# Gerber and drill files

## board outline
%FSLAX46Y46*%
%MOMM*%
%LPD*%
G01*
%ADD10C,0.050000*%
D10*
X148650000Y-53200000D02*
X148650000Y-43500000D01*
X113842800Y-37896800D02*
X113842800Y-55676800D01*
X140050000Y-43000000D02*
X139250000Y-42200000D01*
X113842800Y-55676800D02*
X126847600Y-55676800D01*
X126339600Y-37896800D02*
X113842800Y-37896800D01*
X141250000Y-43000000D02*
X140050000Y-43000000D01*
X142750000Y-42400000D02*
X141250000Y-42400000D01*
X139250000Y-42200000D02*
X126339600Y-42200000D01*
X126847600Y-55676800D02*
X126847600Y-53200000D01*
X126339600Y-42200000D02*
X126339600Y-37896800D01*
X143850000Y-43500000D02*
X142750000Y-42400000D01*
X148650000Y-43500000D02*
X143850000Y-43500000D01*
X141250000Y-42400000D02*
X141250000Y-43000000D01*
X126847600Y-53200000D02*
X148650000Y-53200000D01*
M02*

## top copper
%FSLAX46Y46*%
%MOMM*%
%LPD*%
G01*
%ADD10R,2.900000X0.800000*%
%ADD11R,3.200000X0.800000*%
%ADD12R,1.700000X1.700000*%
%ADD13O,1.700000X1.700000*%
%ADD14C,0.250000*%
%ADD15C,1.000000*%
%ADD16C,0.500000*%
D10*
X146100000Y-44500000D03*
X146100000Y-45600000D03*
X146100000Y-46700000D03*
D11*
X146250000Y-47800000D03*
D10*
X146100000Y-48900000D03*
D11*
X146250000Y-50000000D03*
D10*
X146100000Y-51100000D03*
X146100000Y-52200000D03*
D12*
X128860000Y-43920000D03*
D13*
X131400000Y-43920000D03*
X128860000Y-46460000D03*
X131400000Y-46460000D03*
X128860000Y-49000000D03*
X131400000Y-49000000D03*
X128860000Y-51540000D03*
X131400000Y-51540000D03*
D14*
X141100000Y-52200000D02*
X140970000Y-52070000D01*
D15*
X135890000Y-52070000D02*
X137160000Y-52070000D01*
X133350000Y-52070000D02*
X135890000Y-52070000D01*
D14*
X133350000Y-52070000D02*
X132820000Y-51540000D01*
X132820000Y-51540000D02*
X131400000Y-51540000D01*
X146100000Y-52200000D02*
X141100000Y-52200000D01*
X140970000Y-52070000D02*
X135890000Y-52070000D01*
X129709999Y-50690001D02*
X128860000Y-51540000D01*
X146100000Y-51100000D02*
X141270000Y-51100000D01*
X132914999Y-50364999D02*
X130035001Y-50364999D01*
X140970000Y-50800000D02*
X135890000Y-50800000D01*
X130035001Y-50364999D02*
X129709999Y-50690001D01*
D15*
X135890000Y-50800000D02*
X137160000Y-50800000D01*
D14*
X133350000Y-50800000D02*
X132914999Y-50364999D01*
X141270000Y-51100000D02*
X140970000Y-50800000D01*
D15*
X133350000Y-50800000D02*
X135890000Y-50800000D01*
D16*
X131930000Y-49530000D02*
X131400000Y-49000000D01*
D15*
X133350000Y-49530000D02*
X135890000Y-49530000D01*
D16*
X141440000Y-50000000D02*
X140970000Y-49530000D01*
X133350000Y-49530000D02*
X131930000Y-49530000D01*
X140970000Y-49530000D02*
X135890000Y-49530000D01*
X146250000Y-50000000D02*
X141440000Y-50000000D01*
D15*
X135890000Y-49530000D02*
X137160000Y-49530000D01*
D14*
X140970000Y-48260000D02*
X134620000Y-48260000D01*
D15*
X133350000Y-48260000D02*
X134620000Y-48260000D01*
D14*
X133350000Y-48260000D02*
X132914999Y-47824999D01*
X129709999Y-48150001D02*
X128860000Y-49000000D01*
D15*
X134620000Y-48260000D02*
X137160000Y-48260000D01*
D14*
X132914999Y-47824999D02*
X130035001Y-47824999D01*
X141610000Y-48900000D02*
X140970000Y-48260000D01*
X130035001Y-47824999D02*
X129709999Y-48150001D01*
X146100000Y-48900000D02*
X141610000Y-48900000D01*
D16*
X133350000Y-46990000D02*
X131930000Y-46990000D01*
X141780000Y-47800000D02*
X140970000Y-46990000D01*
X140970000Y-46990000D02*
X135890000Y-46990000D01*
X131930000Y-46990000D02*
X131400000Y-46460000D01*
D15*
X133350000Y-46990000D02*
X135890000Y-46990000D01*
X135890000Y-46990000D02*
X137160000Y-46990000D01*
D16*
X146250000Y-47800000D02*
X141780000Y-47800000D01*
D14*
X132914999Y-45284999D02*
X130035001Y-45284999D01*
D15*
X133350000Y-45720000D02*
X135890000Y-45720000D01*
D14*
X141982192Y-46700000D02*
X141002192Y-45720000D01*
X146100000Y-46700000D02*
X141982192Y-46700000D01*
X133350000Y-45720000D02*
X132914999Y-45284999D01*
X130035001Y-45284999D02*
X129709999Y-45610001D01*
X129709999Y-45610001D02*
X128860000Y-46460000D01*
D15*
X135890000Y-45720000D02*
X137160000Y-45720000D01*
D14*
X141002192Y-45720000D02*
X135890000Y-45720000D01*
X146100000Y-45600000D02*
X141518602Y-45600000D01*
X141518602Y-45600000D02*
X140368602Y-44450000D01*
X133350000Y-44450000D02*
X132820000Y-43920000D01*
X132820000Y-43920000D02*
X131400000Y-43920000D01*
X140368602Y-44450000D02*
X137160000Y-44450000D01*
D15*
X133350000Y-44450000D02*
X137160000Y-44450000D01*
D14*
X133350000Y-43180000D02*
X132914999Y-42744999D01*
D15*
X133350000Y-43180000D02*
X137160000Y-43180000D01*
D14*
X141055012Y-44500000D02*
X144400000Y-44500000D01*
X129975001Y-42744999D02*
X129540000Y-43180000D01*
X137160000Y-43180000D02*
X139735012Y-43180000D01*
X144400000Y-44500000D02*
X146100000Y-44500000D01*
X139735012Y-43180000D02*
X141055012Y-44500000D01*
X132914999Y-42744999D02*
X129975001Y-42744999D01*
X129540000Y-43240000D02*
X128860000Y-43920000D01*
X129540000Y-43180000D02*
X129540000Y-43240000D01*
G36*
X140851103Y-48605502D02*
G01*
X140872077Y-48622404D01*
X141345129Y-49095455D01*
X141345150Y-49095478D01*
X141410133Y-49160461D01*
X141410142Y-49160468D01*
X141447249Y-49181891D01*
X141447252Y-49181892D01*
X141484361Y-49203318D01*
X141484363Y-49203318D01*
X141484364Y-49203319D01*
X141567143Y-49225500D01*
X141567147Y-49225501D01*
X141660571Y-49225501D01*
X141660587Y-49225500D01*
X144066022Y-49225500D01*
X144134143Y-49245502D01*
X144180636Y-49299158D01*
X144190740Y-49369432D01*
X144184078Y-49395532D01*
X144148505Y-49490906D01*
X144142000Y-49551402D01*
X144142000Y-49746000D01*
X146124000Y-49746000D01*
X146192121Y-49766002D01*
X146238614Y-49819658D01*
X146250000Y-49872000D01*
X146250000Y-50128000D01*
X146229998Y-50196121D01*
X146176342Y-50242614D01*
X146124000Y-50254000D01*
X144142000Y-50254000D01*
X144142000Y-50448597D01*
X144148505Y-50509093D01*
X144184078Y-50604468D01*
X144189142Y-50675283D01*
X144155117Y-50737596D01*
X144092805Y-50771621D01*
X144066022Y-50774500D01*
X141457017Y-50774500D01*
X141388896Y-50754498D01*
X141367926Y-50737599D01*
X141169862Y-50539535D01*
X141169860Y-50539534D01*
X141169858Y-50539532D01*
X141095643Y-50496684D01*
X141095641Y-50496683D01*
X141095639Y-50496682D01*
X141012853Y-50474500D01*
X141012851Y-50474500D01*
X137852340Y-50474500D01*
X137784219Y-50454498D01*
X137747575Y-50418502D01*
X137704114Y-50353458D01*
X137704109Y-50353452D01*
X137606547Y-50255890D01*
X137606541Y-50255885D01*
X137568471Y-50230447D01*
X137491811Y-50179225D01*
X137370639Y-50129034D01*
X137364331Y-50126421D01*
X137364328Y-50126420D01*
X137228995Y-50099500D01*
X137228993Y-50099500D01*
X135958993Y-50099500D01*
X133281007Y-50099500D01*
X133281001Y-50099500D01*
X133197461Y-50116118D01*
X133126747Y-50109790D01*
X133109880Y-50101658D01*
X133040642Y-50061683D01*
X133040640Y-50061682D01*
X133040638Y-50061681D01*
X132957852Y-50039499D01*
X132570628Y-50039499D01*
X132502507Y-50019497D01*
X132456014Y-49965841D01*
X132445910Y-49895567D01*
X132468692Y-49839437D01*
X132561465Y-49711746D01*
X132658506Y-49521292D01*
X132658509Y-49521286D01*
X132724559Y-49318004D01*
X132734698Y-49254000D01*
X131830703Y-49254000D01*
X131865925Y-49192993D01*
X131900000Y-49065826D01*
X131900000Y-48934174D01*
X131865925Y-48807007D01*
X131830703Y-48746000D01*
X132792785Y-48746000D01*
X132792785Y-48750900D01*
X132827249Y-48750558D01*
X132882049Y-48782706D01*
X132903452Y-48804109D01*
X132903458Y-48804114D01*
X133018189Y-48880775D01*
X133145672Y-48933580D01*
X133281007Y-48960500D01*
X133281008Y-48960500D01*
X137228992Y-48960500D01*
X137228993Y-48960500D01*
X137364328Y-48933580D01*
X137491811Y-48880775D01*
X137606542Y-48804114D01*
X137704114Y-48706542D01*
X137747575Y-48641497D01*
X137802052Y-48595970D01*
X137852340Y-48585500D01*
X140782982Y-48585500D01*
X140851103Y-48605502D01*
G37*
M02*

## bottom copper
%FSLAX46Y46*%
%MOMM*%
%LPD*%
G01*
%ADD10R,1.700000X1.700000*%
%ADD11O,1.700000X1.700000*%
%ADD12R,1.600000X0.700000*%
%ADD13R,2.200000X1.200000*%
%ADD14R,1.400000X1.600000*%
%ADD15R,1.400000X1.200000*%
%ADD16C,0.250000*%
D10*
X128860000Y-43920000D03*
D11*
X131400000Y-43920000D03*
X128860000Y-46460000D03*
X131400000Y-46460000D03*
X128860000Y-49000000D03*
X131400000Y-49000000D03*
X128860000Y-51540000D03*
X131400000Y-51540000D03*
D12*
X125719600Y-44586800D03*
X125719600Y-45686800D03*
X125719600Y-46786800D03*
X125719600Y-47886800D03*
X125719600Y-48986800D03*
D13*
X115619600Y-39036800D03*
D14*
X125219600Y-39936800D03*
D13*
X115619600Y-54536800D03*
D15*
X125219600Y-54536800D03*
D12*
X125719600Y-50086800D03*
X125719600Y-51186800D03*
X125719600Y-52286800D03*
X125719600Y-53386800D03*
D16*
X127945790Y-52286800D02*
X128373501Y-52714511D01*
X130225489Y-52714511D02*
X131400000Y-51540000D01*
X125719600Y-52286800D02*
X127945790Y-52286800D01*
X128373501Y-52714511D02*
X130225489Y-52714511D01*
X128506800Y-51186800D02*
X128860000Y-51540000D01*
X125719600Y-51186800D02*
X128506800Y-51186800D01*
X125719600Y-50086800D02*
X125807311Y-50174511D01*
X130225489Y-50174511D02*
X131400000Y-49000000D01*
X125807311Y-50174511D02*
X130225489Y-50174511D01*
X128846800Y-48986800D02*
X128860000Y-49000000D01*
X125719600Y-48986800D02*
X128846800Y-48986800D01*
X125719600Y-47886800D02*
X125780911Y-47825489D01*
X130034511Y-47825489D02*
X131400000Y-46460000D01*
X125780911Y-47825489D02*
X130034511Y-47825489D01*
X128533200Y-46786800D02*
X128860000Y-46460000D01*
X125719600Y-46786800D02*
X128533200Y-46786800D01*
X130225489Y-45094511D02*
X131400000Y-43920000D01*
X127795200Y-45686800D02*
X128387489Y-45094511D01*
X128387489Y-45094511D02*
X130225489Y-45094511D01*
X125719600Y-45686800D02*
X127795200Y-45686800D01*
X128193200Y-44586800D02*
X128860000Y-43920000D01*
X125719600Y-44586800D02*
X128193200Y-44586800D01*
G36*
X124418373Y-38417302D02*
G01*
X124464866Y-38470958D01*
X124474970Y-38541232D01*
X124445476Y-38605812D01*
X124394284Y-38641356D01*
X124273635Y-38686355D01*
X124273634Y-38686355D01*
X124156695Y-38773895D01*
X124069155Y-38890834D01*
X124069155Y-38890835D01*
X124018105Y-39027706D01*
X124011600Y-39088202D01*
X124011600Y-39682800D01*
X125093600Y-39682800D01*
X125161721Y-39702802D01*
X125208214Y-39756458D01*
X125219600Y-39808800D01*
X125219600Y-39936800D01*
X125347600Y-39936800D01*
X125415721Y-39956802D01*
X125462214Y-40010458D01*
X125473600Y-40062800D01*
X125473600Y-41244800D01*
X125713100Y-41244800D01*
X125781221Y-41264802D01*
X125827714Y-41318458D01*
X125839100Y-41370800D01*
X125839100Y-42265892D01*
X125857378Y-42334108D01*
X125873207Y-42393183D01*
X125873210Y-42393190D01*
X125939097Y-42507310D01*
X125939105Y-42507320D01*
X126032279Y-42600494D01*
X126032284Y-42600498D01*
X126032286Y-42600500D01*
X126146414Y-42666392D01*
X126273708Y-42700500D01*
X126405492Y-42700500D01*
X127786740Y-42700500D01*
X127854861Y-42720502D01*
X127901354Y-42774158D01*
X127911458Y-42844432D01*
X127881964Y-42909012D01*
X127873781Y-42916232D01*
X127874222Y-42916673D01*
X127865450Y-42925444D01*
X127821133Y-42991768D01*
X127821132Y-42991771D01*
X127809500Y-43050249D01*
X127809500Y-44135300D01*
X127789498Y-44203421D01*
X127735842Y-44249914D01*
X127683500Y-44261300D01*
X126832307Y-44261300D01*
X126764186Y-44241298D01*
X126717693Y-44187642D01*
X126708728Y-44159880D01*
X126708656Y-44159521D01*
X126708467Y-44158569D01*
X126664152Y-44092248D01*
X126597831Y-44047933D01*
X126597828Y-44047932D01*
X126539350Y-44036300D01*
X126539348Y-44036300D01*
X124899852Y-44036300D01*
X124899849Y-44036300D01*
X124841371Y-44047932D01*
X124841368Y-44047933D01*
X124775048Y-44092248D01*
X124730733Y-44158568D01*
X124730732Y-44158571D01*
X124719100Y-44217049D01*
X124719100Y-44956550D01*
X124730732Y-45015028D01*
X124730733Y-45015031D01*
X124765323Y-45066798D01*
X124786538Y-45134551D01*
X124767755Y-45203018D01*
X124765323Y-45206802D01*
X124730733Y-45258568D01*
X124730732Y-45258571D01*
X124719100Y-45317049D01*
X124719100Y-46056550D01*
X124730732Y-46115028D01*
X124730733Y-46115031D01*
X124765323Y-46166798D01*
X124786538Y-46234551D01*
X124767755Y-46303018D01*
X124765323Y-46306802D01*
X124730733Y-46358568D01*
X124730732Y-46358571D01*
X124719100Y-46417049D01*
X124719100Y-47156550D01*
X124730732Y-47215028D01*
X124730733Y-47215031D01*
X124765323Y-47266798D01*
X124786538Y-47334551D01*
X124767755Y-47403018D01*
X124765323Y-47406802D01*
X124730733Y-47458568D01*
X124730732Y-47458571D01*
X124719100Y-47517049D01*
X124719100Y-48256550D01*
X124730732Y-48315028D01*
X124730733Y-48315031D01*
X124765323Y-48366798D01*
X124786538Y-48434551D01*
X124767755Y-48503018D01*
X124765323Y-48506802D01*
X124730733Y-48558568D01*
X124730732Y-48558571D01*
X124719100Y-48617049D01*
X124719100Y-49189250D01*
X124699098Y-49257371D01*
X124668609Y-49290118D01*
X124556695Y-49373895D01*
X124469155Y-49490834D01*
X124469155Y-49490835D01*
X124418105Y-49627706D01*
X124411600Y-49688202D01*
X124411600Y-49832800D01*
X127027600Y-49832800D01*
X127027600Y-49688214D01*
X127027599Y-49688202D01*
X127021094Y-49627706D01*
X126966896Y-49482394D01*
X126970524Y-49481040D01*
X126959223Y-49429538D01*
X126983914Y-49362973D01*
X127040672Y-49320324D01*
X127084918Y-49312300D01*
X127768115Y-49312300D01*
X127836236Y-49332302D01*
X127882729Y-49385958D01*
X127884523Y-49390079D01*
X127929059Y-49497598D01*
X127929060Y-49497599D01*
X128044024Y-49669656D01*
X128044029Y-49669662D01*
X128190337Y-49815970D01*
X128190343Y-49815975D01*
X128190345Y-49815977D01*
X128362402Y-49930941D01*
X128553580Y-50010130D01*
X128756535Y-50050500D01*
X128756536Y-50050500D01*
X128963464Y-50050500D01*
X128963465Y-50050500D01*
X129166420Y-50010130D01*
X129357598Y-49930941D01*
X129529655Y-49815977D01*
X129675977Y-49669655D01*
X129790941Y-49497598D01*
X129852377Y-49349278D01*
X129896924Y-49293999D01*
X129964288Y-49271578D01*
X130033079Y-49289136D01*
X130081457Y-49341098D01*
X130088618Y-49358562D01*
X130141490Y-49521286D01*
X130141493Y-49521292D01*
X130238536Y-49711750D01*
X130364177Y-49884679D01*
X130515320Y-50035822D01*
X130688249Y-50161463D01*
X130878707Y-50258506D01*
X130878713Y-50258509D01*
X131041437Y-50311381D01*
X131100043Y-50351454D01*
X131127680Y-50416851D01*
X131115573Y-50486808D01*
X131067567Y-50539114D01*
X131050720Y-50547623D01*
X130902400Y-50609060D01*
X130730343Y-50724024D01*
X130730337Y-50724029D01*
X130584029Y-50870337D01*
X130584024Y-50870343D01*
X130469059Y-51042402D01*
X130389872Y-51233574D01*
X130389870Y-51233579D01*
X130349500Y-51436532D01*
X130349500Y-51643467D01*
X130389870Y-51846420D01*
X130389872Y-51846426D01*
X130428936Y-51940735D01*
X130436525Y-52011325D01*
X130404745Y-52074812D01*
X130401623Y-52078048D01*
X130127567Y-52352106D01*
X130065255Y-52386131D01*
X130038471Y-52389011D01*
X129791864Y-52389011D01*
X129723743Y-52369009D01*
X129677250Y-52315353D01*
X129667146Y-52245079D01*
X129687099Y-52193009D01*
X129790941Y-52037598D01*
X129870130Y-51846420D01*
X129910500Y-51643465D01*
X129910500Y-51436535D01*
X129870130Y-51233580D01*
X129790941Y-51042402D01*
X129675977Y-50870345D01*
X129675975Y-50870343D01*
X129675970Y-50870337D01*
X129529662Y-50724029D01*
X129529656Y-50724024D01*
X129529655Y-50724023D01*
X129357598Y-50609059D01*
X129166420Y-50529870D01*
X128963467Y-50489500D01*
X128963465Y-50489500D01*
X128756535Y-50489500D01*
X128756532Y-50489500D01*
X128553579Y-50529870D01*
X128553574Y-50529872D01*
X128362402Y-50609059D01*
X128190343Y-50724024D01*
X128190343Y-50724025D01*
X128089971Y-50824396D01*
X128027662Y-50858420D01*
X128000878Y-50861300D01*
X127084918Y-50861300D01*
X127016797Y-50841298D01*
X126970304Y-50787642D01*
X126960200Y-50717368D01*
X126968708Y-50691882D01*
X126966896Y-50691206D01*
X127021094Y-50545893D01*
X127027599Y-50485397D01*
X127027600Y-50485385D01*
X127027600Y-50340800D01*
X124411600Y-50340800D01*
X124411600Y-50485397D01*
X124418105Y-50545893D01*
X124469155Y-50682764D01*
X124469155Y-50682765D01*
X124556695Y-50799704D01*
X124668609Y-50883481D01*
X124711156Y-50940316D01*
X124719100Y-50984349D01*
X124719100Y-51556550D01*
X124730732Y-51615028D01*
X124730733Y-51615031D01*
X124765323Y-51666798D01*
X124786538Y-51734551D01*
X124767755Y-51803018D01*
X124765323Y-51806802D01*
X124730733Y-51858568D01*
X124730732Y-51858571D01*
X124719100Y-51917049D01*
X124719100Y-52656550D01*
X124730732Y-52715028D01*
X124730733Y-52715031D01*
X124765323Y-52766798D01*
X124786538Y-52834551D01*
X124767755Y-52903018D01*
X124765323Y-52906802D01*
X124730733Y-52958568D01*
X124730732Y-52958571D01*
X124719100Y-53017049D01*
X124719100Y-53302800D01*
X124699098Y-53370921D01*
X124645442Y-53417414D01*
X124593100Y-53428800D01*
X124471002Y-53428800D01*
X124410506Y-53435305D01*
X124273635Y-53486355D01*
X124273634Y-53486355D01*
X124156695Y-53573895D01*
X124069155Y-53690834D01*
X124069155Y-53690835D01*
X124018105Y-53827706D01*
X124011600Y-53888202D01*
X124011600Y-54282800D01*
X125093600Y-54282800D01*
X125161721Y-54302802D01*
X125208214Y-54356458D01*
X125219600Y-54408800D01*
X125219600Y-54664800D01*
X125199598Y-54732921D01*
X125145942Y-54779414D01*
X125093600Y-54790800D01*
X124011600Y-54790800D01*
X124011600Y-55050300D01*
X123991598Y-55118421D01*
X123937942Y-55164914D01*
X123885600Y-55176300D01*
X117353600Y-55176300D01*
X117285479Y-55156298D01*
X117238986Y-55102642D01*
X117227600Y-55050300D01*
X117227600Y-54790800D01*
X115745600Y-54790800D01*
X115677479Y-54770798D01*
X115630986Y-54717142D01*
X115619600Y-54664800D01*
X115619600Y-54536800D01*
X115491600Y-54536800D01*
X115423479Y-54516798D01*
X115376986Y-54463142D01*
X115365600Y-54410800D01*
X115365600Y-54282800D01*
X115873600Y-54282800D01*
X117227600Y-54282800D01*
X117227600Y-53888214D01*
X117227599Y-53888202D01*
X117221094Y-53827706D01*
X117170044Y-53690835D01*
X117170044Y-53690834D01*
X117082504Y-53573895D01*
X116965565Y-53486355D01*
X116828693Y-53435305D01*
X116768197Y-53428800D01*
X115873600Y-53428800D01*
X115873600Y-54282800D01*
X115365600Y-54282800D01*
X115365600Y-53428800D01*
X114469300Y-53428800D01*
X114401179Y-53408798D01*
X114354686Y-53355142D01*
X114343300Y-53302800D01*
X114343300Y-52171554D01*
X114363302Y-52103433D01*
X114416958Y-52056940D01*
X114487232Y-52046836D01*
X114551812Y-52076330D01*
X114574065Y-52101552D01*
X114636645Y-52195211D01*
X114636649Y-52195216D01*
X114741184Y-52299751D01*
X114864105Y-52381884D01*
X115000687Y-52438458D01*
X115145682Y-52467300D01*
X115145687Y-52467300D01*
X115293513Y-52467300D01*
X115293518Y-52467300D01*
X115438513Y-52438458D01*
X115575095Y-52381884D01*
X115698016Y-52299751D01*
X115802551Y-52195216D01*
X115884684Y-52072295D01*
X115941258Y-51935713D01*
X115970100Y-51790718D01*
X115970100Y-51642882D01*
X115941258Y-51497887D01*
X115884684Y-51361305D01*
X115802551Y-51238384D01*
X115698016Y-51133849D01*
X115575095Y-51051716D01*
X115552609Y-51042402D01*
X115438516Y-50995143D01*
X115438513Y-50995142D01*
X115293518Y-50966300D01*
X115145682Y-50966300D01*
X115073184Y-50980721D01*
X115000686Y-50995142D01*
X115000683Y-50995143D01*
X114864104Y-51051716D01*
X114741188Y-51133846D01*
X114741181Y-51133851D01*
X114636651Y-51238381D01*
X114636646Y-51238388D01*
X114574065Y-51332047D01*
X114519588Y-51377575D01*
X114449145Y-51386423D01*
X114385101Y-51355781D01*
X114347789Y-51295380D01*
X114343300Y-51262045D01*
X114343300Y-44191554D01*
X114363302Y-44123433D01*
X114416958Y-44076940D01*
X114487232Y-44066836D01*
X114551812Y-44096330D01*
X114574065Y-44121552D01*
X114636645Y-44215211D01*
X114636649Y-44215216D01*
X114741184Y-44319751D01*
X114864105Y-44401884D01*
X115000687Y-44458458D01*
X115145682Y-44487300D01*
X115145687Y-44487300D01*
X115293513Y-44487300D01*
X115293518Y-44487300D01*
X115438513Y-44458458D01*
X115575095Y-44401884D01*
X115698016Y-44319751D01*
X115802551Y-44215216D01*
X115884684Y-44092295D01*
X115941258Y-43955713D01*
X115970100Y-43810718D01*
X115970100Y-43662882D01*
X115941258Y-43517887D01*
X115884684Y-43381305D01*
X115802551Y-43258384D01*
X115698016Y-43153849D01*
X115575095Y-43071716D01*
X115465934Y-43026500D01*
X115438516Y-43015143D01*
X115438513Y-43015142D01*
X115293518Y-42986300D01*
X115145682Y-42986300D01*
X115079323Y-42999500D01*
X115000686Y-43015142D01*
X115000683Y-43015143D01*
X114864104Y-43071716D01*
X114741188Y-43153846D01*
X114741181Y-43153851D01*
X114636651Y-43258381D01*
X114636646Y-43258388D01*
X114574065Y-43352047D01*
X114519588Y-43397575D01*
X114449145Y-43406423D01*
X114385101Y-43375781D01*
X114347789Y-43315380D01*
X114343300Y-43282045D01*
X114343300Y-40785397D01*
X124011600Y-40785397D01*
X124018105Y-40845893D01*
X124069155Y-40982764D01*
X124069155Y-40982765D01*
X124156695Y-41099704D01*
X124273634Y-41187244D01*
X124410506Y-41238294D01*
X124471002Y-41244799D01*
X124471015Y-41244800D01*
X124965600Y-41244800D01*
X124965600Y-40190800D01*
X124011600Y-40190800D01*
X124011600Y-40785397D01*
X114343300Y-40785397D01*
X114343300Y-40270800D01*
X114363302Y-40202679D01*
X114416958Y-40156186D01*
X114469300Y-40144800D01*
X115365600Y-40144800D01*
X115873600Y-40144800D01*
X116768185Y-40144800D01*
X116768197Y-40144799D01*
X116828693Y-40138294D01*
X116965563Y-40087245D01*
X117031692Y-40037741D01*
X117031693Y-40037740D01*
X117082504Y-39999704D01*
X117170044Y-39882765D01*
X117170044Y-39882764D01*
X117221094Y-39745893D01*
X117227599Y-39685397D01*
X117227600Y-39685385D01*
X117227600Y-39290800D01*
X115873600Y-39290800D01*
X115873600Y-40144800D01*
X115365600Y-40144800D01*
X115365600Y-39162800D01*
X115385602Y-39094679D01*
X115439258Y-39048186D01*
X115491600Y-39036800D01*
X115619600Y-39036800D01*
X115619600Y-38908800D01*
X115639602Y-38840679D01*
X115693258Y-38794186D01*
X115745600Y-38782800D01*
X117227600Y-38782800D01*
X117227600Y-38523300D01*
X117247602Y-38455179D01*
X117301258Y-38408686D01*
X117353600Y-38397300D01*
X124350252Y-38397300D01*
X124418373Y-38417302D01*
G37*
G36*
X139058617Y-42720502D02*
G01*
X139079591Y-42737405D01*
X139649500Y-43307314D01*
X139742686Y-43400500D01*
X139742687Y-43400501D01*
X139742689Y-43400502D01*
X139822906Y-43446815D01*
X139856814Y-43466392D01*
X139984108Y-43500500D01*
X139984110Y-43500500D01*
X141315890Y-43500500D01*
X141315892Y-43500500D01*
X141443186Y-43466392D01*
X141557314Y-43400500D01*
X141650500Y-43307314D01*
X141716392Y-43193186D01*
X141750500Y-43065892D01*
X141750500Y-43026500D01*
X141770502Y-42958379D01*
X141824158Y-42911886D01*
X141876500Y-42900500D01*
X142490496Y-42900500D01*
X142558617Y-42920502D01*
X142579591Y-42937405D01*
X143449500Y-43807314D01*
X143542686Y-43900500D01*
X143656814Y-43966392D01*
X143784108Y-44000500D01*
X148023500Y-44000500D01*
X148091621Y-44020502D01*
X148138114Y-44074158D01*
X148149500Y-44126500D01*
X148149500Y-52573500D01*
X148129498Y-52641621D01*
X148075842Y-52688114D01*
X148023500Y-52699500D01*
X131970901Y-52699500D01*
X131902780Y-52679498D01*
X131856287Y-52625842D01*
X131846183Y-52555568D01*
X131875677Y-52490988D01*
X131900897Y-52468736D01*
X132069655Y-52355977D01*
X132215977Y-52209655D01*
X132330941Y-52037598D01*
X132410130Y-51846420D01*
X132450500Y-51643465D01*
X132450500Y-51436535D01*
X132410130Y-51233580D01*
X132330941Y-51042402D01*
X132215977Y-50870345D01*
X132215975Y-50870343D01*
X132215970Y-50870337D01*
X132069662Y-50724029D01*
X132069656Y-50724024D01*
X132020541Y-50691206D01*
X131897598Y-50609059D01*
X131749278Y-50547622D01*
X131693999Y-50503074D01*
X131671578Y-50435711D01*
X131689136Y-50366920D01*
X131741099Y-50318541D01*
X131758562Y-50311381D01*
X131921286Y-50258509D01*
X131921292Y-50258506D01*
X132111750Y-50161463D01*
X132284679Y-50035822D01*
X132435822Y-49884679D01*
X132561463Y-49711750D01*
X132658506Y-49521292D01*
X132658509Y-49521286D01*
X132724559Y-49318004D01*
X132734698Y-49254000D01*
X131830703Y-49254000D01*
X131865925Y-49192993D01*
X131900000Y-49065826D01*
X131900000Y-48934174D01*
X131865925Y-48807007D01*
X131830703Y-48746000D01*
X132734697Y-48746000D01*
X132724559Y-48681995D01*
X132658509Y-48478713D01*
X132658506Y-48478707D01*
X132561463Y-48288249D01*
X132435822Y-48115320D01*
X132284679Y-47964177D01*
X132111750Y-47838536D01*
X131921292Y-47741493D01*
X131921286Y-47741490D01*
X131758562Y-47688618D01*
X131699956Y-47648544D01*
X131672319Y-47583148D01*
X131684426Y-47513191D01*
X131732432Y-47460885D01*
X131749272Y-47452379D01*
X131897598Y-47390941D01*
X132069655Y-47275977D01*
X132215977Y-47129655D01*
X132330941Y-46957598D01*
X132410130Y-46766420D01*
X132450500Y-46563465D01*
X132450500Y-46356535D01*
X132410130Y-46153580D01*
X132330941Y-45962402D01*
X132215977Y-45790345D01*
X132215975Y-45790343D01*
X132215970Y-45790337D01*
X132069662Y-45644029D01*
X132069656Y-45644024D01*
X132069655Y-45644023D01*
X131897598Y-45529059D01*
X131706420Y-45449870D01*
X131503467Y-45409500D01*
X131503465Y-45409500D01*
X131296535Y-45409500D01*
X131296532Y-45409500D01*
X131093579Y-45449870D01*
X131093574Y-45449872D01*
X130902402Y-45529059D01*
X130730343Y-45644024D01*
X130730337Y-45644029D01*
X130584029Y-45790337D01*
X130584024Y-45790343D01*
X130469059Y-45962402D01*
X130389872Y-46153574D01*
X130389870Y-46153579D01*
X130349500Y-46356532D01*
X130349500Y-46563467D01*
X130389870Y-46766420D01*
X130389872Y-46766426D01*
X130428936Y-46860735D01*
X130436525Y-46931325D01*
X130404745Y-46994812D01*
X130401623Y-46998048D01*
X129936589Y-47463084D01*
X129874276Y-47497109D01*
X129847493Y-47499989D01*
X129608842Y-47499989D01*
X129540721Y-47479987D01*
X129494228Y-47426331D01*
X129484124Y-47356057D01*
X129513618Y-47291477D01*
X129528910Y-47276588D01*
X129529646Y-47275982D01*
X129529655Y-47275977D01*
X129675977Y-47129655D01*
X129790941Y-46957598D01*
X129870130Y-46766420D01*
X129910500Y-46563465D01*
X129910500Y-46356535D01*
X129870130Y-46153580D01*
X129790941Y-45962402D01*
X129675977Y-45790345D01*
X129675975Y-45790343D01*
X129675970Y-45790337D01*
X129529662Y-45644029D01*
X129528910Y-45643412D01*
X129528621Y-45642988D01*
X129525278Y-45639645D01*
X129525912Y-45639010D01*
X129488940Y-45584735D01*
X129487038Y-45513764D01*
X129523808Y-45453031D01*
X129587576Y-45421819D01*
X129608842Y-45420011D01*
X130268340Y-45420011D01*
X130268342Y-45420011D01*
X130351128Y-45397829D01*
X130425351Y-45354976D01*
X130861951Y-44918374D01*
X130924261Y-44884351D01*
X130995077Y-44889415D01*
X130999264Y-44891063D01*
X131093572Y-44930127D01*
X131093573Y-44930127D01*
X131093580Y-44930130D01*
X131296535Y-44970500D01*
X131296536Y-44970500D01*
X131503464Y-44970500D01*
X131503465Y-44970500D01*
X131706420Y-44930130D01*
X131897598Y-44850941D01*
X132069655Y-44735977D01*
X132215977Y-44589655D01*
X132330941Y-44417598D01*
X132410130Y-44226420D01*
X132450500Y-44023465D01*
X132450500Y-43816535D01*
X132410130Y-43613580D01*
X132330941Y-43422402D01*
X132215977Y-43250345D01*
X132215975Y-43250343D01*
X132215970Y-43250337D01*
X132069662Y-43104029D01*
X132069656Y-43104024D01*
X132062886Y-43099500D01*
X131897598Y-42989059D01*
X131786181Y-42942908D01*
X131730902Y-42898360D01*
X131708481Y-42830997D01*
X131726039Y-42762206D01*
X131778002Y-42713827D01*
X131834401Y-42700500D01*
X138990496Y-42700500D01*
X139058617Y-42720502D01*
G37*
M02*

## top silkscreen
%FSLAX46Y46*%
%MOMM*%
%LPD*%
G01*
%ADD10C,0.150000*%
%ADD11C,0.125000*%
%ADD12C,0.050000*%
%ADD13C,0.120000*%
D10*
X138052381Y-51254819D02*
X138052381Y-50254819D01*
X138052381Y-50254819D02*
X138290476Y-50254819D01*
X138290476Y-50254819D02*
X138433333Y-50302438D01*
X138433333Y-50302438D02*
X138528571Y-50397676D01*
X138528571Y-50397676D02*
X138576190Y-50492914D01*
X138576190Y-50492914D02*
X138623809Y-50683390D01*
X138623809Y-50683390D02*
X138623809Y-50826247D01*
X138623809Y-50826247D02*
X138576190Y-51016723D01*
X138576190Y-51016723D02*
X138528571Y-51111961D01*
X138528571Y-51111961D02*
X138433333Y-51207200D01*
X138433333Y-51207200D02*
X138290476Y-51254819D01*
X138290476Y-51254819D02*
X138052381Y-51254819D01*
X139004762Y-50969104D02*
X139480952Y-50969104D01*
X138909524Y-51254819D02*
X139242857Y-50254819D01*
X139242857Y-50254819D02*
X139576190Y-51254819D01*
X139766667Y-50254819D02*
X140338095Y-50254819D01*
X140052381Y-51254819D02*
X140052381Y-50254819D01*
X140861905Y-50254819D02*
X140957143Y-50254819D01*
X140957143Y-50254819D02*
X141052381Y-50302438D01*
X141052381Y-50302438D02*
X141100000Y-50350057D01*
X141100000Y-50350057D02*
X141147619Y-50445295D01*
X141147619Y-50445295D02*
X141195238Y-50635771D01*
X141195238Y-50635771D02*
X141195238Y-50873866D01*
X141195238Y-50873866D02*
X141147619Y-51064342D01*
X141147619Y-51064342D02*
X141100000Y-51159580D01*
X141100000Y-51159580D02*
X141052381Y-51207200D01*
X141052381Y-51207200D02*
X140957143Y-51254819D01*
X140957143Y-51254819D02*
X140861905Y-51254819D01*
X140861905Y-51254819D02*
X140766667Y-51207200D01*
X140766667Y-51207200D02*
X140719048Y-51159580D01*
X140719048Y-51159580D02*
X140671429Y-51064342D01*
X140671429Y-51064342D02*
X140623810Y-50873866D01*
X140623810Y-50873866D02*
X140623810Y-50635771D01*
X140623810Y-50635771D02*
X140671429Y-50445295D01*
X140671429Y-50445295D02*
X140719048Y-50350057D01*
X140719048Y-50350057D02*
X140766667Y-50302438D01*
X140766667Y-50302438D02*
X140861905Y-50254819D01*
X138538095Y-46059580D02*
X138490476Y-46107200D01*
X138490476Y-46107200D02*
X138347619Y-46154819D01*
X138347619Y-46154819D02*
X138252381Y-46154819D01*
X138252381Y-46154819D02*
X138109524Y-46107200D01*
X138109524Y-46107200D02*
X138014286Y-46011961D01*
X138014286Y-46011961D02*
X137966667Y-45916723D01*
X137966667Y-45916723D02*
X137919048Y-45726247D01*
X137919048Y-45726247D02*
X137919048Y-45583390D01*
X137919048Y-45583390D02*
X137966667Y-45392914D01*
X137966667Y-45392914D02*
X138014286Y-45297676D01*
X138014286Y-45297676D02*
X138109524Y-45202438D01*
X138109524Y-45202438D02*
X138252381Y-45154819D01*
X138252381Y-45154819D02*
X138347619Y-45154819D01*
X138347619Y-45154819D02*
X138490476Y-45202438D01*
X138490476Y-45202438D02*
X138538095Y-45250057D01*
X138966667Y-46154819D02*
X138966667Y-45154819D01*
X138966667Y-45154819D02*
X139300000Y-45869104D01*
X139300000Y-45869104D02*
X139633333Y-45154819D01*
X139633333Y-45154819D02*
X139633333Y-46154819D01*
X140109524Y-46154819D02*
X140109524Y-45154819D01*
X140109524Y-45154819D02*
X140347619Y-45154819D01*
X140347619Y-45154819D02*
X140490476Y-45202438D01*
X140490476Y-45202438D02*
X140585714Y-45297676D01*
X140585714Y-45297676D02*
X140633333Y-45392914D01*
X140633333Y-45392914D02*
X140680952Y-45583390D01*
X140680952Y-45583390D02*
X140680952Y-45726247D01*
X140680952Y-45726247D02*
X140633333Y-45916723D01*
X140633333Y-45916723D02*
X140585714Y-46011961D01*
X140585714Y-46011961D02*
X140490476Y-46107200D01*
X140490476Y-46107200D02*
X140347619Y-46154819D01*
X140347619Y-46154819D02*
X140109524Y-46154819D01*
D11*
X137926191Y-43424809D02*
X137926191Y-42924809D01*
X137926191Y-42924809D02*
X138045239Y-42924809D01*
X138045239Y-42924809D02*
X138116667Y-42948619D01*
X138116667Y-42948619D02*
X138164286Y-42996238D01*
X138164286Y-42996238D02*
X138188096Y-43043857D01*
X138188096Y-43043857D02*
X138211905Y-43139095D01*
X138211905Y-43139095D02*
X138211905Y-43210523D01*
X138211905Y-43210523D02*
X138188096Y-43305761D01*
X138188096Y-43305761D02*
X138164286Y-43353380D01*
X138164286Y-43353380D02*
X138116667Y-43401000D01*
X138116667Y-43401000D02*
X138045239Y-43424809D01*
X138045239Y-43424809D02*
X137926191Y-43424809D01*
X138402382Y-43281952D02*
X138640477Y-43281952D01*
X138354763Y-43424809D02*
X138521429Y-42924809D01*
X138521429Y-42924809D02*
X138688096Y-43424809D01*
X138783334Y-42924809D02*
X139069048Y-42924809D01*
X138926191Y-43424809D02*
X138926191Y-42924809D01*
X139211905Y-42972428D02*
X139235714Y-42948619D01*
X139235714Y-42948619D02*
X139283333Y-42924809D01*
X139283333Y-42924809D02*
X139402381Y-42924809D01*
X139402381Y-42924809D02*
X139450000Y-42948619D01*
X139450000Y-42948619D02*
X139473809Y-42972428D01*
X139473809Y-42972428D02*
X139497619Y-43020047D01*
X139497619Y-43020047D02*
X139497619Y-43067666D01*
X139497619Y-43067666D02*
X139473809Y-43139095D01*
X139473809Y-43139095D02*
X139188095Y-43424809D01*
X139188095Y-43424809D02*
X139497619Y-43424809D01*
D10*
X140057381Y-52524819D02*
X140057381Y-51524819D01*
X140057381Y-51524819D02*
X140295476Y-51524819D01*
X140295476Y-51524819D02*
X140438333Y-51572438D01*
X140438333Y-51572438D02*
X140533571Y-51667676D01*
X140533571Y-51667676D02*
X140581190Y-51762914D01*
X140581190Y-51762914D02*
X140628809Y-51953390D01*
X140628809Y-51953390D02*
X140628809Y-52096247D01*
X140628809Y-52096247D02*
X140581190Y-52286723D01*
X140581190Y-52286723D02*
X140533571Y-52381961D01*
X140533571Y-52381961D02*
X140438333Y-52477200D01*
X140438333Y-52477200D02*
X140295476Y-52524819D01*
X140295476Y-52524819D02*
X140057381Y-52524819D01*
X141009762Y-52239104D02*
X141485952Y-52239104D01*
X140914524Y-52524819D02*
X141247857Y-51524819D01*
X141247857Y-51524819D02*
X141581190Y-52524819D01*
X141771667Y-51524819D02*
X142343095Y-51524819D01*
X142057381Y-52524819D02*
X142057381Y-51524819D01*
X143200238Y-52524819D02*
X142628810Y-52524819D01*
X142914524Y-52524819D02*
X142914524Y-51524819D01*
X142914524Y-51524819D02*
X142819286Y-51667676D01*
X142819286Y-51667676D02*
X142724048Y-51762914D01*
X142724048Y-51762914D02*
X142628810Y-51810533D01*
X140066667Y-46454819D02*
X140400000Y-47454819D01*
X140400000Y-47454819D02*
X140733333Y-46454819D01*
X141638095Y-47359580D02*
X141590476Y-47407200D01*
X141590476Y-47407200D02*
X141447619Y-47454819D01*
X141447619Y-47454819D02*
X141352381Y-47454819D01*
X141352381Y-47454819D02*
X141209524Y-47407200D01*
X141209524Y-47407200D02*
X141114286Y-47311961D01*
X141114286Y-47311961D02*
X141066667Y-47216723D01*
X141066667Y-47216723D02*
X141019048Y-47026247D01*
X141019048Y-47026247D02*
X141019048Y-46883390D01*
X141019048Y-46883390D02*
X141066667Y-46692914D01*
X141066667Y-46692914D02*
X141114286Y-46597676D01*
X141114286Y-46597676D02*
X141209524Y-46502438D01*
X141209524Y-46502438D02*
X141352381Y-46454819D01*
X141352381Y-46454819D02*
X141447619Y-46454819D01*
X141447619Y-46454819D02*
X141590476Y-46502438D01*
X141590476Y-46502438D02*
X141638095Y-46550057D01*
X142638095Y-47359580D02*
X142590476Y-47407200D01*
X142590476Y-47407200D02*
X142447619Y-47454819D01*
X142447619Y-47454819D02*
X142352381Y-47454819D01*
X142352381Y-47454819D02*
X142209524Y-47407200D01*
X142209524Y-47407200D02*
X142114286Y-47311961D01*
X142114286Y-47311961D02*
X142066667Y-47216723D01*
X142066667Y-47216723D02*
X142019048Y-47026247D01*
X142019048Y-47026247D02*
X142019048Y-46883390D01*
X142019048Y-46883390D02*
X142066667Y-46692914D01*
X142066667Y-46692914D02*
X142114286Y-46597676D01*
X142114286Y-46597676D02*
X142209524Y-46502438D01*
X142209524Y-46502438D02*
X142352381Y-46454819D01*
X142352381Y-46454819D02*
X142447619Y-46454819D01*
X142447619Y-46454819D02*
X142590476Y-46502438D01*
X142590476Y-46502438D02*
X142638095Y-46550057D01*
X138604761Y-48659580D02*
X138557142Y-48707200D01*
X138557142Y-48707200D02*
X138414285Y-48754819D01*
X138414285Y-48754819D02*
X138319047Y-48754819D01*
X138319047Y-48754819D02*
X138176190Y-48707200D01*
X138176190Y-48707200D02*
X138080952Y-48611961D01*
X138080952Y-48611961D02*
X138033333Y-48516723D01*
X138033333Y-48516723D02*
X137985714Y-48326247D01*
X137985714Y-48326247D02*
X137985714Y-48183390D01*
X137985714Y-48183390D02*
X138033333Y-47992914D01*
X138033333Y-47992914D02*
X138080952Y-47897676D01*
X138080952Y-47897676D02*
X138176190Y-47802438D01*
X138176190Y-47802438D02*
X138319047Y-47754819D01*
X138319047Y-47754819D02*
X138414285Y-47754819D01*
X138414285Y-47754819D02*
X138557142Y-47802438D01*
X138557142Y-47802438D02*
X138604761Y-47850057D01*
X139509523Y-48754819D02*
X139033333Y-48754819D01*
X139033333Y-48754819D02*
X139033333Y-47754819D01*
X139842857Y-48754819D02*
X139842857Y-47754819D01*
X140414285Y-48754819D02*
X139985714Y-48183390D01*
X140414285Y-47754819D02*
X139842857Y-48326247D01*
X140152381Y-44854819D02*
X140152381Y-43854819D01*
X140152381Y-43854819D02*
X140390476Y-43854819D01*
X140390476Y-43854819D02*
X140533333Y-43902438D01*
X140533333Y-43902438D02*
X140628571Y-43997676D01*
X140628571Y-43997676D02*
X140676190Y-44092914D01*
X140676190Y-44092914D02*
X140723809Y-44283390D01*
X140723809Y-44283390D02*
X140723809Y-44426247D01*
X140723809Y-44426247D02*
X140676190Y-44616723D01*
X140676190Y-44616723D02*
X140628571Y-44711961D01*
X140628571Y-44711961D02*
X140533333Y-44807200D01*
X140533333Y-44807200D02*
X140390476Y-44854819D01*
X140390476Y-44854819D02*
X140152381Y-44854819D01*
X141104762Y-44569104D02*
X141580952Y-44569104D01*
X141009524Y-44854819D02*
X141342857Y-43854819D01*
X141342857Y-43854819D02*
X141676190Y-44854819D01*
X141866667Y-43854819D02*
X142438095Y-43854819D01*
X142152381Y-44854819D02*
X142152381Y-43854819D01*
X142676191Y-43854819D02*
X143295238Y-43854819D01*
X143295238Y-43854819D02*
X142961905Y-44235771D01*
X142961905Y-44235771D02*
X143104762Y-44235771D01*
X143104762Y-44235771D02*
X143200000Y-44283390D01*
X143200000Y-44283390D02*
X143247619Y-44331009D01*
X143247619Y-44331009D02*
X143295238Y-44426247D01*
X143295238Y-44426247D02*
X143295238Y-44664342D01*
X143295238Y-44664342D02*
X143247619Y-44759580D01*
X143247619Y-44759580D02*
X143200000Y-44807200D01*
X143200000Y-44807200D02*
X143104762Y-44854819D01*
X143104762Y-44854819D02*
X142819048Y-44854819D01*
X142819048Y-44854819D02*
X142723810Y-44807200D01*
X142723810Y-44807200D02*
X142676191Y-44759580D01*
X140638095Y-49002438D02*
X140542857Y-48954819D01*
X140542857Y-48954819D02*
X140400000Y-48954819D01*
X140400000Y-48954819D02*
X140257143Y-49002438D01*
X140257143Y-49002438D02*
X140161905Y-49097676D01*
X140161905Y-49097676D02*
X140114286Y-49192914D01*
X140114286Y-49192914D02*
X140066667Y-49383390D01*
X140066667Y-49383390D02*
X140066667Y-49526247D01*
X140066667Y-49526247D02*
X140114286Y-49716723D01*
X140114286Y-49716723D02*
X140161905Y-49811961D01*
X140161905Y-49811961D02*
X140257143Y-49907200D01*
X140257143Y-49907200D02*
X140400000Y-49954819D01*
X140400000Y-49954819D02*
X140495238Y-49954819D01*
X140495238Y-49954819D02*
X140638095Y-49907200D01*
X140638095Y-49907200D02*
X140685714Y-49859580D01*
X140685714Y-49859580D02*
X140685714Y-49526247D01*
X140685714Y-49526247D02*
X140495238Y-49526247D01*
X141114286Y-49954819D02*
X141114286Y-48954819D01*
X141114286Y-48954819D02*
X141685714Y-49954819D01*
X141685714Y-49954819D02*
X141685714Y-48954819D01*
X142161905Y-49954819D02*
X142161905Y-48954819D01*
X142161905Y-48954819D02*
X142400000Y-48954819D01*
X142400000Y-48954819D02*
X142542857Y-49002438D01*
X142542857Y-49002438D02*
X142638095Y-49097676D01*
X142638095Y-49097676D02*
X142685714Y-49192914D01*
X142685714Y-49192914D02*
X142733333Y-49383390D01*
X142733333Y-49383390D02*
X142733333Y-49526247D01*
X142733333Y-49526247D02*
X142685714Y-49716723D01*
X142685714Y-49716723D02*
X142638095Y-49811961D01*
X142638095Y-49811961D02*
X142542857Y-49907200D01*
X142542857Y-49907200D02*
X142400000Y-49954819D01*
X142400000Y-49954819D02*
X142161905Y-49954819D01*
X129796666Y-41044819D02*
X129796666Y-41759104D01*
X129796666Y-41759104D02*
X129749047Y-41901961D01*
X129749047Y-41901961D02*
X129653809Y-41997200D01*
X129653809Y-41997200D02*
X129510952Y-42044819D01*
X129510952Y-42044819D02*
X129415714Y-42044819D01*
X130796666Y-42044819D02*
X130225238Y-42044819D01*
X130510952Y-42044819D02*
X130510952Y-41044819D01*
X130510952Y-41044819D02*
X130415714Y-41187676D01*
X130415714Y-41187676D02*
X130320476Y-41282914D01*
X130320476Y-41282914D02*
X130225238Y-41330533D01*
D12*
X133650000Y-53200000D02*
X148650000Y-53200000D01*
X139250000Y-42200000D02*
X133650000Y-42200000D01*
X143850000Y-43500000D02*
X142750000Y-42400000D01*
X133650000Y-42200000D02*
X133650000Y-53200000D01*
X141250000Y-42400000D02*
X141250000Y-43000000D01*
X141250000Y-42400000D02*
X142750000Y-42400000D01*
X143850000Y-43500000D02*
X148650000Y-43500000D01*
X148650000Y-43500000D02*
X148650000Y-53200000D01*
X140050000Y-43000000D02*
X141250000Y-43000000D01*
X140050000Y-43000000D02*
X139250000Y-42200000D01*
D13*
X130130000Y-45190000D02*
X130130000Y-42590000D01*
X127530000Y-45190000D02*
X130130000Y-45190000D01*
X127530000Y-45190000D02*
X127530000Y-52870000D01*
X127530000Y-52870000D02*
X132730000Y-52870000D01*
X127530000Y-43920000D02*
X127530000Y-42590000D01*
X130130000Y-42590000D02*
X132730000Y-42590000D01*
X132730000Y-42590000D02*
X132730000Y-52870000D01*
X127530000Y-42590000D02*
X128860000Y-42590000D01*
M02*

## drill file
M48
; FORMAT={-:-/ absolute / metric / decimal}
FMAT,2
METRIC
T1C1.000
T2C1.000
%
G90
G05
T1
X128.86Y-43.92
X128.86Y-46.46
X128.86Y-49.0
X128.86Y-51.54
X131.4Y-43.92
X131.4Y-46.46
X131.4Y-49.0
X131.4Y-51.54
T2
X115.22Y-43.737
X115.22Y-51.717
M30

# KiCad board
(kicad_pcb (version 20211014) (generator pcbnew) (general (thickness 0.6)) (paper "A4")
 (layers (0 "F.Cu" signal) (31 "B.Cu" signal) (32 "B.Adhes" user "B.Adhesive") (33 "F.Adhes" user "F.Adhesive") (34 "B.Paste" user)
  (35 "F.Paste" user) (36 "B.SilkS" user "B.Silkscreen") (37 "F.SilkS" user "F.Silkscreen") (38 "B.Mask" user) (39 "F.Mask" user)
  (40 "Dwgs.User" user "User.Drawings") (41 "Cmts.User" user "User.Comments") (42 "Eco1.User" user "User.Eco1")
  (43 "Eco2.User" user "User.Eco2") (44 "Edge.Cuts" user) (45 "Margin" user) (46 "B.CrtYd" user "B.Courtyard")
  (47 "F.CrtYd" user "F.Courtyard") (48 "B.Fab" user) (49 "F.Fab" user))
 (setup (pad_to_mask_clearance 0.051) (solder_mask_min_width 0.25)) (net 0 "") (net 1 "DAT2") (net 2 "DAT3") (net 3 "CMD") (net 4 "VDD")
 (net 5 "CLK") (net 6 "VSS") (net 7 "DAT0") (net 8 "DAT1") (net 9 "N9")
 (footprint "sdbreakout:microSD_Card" (layer "F.Cu") (at 141.15 48.3)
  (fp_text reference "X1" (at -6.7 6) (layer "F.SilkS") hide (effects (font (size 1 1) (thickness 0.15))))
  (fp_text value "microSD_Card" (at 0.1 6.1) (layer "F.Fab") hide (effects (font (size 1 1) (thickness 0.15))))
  (fp_line (start -7.5 4.9) (end 7.5 4.9) (layer "F.SilkS") (width 0.05))
  (fp_line (start -1.9 -6.1) (end -7.5 -6.1) (layer "F.SilkS") (width 0.05))
  (fp_line (start 2.7 -4.8) (end 1.6 -5.9) (layer "F.SilkS") (width 0.05))
  (fp_line (start -7.5 -6.1) (end -7.5 4.9) (layer "F.SilkS") (width 0.05))
  (fp_line (start 0.1 -5.9) (end 0.1 -5.3) (layer "F.SilkS") (width 0.05))
  (fp_line (start 0.1 -5.9) (end 1.6 -5.9) (layer "F.SilkS") (width 0.05))
  (fp_line (start 2.7 -4.8) (end 7.5 -4.8) (layer "F.SilkS") (width 0.05))
  (fp_line (start 7.5 -4.8) (end 7.5 4.9) (layer "F.SilkS") (width 0.05))
  (fp_line (start -1.1 -5.3) (end 0.1 -5.3) (layer "F.SilkS") (width 0.05))
  (fp_line (start -1.1 -5.3) (end -1.9 -6.1) (layer "F.SilkS") (width 0.05))
  (pad "1" smd rect locked (at 4.95 -3.8 90) (size 0.8 2.9) (layers "F.Cu" "F.Paste" "F.Mask") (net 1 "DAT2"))
  (pad "2" smd rect locked (at 4.95 -2.7 90) (size 0.8 2.9) (layers "F.Cu" "F.Paste" "F.Mask") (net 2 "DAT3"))
  (pad "3" smd rect locked (at 4.95 -1.6 90) (size 0.8 2.9) (layers "F.Cu" "F.Paste" "F.Mask") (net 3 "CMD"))
  (pad "4" smd rect locked (at 5.1 -0.5 90) (size 0.8 3.2) (layers "F.Cu" "F.Paste" "F.Mask") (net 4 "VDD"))
  (pad "5" smd rect locked (at 4.95 0.6 90) (size 0.8 2.9) (layers "F.Cu" "F.Paste" "F.Mask") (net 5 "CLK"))
  (pad "6" smd rect locked (at 5.1 1.7 90) (size 0.8 3.2) (layers "F.Cu" "F.Paste" "F.Mask") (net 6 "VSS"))
  (pad "7" smd rect locked (at 4.95 2.8 90) (size 0.8 2.9) (layers "F.Cu" "F.Paste" "F.Mask") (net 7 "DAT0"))
  (pad "8" smd rect locked (at 4.95 3.9 90) (size 0.8 2.9) (layers "F.Cu" "F.Paste" "F.Mask") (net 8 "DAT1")))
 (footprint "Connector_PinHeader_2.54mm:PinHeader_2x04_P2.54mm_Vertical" (layer "F.Cu") (at 128.86 43.92)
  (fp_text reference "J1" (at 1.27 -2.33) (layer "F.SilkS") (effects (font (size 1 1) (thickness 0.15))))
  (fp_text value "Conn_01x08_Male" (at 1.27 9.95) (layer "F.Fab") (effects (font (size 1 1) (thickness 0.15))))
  (fp_line (start 1.27 1.27) (end 1.27 -1.33) (layer "F.SilkS") (width 0.12))
  (fp_line (start -1.33 1.27) (end 1.27 1.27) (layer "F.SilkS") (width 0.12))
  (fp_line (start -1.33 1.27) (end -1.33 8.95) (layer "F.SilkS") (width 0.12))
  (fp_line (start -1.33 8.95) (end 3.87 8.95) (layer "F.SilkS") (width 0.12))
  (fp_line (start -1.33 0) (end -1.33 -1.33) (layer "F.SilkS") (width 0.12))
  (fp_line (start 1.27 -1.33) (end 3.87 -1.33) (layer "F.SilkS") (width 0.12))
  (fp_line (start 3.87 -1.33) (end 3.87 8.95) (layer "F.SilkS") (width 0.12))
  (fp_line (start -1.33 -1.33) (end 0 -1.33) (layer "F.SilkS") (width 0.12))
  (pad "1" thru_hole rect locked (at 0 0) (size 1.7 1.7) (drill 1) (layers *.Cu *.Mask) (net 1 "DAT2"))
  (pad "2" thru_hole oval locked (at 2.54 0) (size 1.7 1.7) (drill 1) (layers *.Cu *.Mask) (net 2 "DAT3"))
  (pad "3" thru_hole oval locked (at 0 2.54) (size 1.7 1.7) (drill 1) (layers *.Cu *.Mask) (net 3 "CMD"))
  (pad "4" thru_hole oval locked (at 2.54 2.54) (size 1.7 1.7) (drill 1) (layers *.Cu *.Mask) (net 4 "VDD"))
  (pad "5" thru_hole oval locked (at 0 5.08) (size 1.7 1.7) (drill 1) (layers *.Cu *.Mask) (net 5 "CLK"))
  (pad "6" thru_hole oval locked (at 2.54 5.08) (size 1.7 1.7) (drill 1) (layers *.Cu *.Mask) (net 6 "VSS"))
  (pad "7" thru_hole oval locked (at 0 7.62) (size 1.7 1.7) (drill 1) (layers *.Cu *.Mask) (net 7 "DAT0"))
  (pad "8" thru_hole oval locked (at 2.54 7.62) (size 1.7 1.7) (drill 1) (layers *.Cu *.Mask) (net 8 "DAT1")))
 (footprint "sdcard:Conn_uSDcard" (layer "B.Cu") (at 118.7196 46.7868 90)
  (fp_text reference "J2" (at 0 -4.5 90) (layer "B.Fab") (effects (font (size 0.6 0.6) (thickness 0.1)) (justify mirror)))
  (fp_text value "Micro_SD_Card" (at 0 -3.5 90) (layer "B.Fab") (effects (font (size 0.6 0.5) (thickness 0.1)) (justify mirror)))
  (pad "" np_thru_hole circle locked (at 3.05 -3.5 90) (size 1 1) (drill 1) (layers *.Cu))
  (pad "" np_thru_hole circle locked (at -4.93 -3.5 90) (size 1 1) (drill 1) (layers *.Cu))
  (pad "1" smd rect locked (at 2.2 7 90) (size 0.7 1.6) (layers "B.Cu" "B.Paste" "B.Mask") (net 1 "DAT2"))
  (pad "2" smd rect locked (at 1.1 7 90) (size 0.7 1.6) (layers "B.Cu" "B.Paste" "B.Mask") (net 2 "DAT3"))
  (pad "3" smd rect locked (at 0 7 90) (size 0.7 1.6) (layers "B.Cu" "B.Paste" "B.Mask") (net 3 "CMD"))
  (pad "4" smd rect locked (at -1.1 7 90) (size 0.7 1.6) (layers "B.Cu" "B.Paste" "B.Mask") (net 4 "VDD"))
  (pad "5" smd rect locked (at -2.2 7 90) (size 0.7 1.6) (layers "B.Cu" "B.Paste" "B.Mask") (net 5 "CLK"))
  (pad "6" smd rect locked (at 7.75 -3.1 90) (size 1.2 2.2) (layers "B.Cu" "B.Paste" "B.Mask") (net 6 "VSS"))
  (pad "6" smd rect locked (at 6.85 6.5 90) (size 1.6 1.4) (layers "B.Cu" "B.Paste" "B.Mask") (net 6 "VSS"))
  (pad "6" smd rect locked (at -7.75 -3.1 90) (size 1.2 2.2) (layers "B.Cu" "B.Paste" "B.Mask") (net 6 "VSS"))
  (pad "6" smd rect locked (at -7.75 6.5 90) (size 1.2 1.4) (layers "B.Cu" "B.Paste" "B.Mask") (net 6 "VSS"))
  (pad "6" smd rect locked (at -3.3 7 90) (size 0.7 1.6) (layers "B.Cu" "B.Paste" "B.Mask") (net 6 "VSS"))
  (pad "7" smd rect locked (at -4.4 7 90) (size 0.7 1.6) (layers "B.Cu" "B.Paste" "B.Mask") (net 7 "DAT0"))
  (pad "8" smd rect locked (at -5.5 7 90) (size 0.7 1.6) (layers "B.Cu" "B.Paste" "B.Mask") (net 8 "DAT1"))
  (pad "9" smd rect locked (at -6.6 7 90) (size 0.7 1.6) (layers "B.Cu" "B.Paste" "B.Mask") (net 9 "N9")))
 (gr_line (start 148.65 53.2) (end 148.65 43.5) (layer "Edge.Cuts") (width 0.05))
 (gr_line (start 113.8428 37.8968) (end 113.8428 55.6768) (layer "Edge.Cuts") (width 0.05))
 (gr_line (start 140.05 43) (end 139.25 42.2) (layer "Edge.Cuts") (width 0.05))
 (gr_line (start 113.8428 55.6768) (end 126.8476 55.6768) (layer "Edge.Cuts") (width 0.05))
 (gr_line (start 126.3396 37.8968) (end 113.8428 37.8968) (layer "Edge.Cuts") (width 0.05))
 (gr_line (start 141.25 43) (end 140.05 43) (layer "Edge.Cuts") (width 0.05))
 (gr_line (start 142.75 42.4) (end 141.25 42.4) (layer "Edge.Cuts") (width 0.05))
 (gr_line (start 139.25 42.2) (end 126.3396 42.2) (layer "Edge.Cuts") (width 0.05))
 (gr_line (start 126.8476 55.6768) (end 126.8476 53.2) (layer "Edge.Cuts") (width 0.05))
 (gr_line (start 126.3396 42.2) (end 126.3396 37.8968) (layer "Edge.Cuts") (width 0.05))
 (gr_line (start 143.85 43.5) (end 142.75 42.4) (layer "Edge.Cuts") (width 0.05))
 (gr_line (start 148.65 43.5) (end 143.85 43.5) (layer "Edge.Cuts") (width 0.05))
 (gr_line (start 141.25 42.4) (end 141.25 43) (layer "Edge.Cuts") (width 0.05))
 (gr_line (start 126.8476 53.2) (end 148.65 53.2) (layer "Edge.Cuts") (width 0.05))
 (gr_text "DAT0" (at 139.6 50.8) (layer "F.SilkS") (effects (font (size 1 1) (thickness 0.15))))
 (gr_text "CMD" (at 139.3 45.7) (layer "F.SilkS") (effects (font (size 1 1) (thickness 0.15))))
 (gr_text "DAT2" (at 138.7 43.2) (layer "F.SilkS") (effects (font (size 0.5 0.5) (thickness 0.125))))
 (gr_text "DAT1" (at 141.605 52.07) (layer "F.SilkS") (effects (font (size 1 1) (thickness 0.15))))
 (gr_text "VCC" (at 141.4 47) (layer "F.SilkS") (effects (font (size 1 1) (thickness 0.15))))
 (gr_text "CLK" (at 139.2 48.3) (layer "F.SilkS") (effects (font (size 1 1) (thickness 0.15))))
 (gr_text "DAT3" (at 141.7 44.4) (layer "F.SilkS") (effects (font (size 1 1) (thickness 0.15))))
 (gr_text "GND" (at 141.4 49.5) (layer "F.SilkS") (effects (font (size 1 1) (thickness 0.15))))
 (segment (start 141.1 52.2) (end 140.97 52.07) (width 0.25) (layer "F.Cu") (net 8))
 (segment (start 135.89 52.07) (end 137.16 52.07) (width 1) (layer "F.Cu") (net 8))
 (segment (start 133.35 52.07) (end 135.89 52.07) (width 1) (layer "F.Cu") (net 8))
 (segment (start 133.35 52.07) (end 132.82 51.54) (width 0.25) (layer "F.Cu") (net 8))
 (segment (start 132.82 51.54) (end 131.4 51.54) (width 0.25) (layer "F.Cu") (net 8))
 (segment (start 146.1 52.2) (end 141.1 52.2) (width 0.25) (layer "F.Cu") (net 8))
 (segment (start 140.97 52.07) (end 135.89 52.07) (width 0.25) (layer "F.Cu") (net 8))
 (segment (start 127.94579 52.2868) (end 128.373501 52.714511) (width 0.25) (layer "B.Cu") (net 8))
 (segment (start 130.225489 52.714511) (end 131.4 51.54) (width 0.25) (layer "B.Cu") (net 8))
 (segment (start 125.7196 52.2868) (end 127.94579 52.2868) (width 0.25) (layer "B.Cu") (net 8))
 (segment (start 128.373501 52.714511) (end 130.225489 52.714511) (width 0.25) (layer "B.Cu") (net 8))
 (segment (start 129.709999 50.690001) (end 128.86 51.54) (width 0.25) (layer "F.Cu") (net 7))
 (segment (start 146.1 51.1) (end 141.27 51.1) (width 0.25) (layer "F.Cu") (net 7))
 (segment (start 132.914999 50.364999) (end 130.035001 50.364999) (width 0.25) (layer "F.Cu") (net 7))
 (segment (start 140.97 50.8) (end 135.89 50.8) (width 0.25) (layer "F.Cu") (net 7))
 (segment (start 130.035001 50.364999) (end 129.709999 50.690001) (width 0.25) (layer "F.Cu") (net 7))
 (segment (start 135.89 50.8) (end 137.16 50.8) (width 1) (layer "F.Cu") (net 7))
 (segment (start 133.35 50.8) (end 132.914999 50.364999) (width 0.25) (layer "F.Cu") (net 7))
 (segment (start 141.27 51.1) (end 140.97 50.8) (width 0.25) (layer "F.Cu") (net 7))
 (segment (start 133.35 50.8) (end 135.89 50.8) (width 1) (layer "F.Cu") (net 7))
 (segment (start 128.5068 51.1868) (end 128.86 51.54) (width 0.25) (layer "B.Cu") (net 7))
 (segment (start 125.7196 51.1868) (end 128.5068 51.1868) (width 0.25) (layer "B.Cu") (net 7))
 (segment (start 131.93 49.53) (end 131.4 49) (width 0.5) (layer "F.Cu") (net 6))
 (segment (start 133.35 49.53) (end 135.89 49.53) (width 1) (layer "F.Cu") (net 6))
 (segment (start 141.44 50) (end 140.97 49.53) (width 0.5) (layer "F.Cu") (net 6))
 (segment (start 133.35 49.53) (end 131.93 49.53) (width 0.5) (layer "F.Cu") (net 6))
 (segment (start 140.97 49.53) (end 135.89 49.53) (width 0.5) (layer "F.Cu") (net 6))
 (segment (start 146.25 50) (end 141.44 50) (width 0.5) (layer "F.Cu") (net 6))
 (segment (start 135.89 49.53) (end 137.16 49.53) (width 1) (layer "F.Cu") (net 6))
 (segment (start 125.7196 50.0868) (end 125.807311 50.174511) (width 0.25) (layer "B.Cu") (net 6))
 (segment (start 130.225489 50.174511) (end 131.4 49) (width 0.25) (layer "B.Cu") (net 6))
 (segment (start 125.807311 50.174511) (end 130.225489 50.174511) (width 0.25) (layer "B.Cu") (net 6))
 (segment (start 140.97 48.26) (end 134.62 48.26) (width 0.25) (layer "F.Cu") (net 5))
 (segment (start 133.35 48.26) (end 134.62 48.26) (width 1) (layer "F.Cu") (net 5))
 (segment (start 133.35 48.26) (end 132.914999 47.824999) (width 0.25) (layer "F.Cu") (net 5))
 (segment (start 129.709999 48.150001) (end 128.86 49) (width 0.25) (layer "F.Cu") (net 5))
 (segment (start 134.62 48.26) (end 137.16 48.26) (width 1) (layer "F.Cu") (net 5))
 (segment (start 132.914999 47.824999) (end 130.035001 47.824999) (width 0.25) (layer "F.Cu") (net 5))
 (segment (start 141.61 48.9) (end 140.97 48.26) (width 0.25) (layer "F.Cu") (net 5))
 (segment (start 130.035001 47.824999) (end 129.709999 48.150001) (width 0.25) (layer "F.Cu") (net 5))
 (segment (start 146.1 48.9) (end 141.61 48.9) (width 0.25) (layer "F.Cu") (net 5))
 (segment (start 128.8468 48.9868) (end 128.86 49) (width 0.25) (layer "B.Cu") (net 5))
 (segment (start 125.7196 48.9868) (end 128.8468 48.9868) (width 0.25) (layer "B.Cu") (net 5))
 (segment (start 133.35 46.99) (end 131.93 46.99) (width 0.5) (layer "F.Cu") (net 4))
 (segment (start 141.78 47.8) (end 140.97 46.99) (width 0.5) (layer "F.Cu") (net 4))
 (segment (start 140.97 46.99) (end 135.89 46.99) (width 0.5) (layer "F.Cu") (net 4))
 (segment (start 131.93 46.99) (end 131.4 46.46) (width 0.5) (layer "F.Cu") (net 4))
 (segment (start 133.35 46.99) (end 135.89 46.99) (width 1) (layer "F.Cu") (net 4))
 (segment (start 135.89 46.99) (end 137.16 46.99) (width 1) (layer "F.Cu") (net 4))
 (segment (start 146.25 47.8) (end 141.78 47.8) (width 0.5) (layer "F.Cu") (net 4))
 (segment (start 125.7196 47.8868) (end 125.780911 47.825489) (width 0.25) (layer "B.Cu") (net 4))
 (segment (start 130.034511 47.825489) (end 131.4 46.46) (width 0.25) (layer "B.Cu") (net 4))
 (segment (start 125.780911 47.825489) (end 130.034511 47.825489) (width 0.25) (layer "B.Cu") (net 4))
 (segment (start 132.914999 45.284999) (end 130.035001 45.284999) (width 0.25) (layer "F.Cu") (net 3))
 (segment (start 133.35 45.72) (end 135.89 45.72) (width 1) (layer "F.Cu") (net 3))
 (segment (start 141.982192 46.7) (end 141.002192 45.72) (width 0.25) (layer "F.Cu") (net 3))
 (segment (start 146.1 46.7) (end 141.982192 46.7) (width 0.25) (layer "F.Cu") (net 3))
 (segment (start 133.35 45.72) (end 132.914999 45.284999) (width 0.25) (layer "F.Cu") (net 3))
 (segment (start 130.035001 45.284999) (end 129.709999 45.610001) (width 0.25) (layer "F.Cu") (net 3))
 (segment (start 129.709999 45.610001) (end 128.86 46.46) (width 0.25) (layer "F.Cu") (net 3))
 (segment (start 135.89 45.72) (end 137.16 45.72) (width 1) (layer "F.Cu") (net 3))
 (segment (start 141.002192 45.72) (end 135.89 45.72) (width 0.25) (layer "F.Cu") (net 3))
 (segment (start 128.5332 46.7868) (end 128.86 46.46) (width 0.25) (layer "B.Cu") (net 3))
 (segment (start 125.7196 46.7868) (end 128.5332 46.7868) (width 0.25) (layer "B.Cu") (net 3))
 (segment (start 146.1 45.6) (end 141.518602 45.6) (width 0.25) (layer "F.Cu") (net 2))
 (segment (start 141.518602 45.6) (end 140.368602 44.45) (width 0.25) (layer "F.Cu") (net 2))
 (segment (start 133.35 44.45) (end 132.82 43.92) (width 0.25) (layer "F.Cu") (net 2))
 (segment (start 132.82 43.92) (end 131.4 43.92) (width 0.25) (layer "F.Cu") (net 2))
 (segment (start 140.368602 44.45) (end 137.16 44.45) (width 0.25) (layer "F.Cu") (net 2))
 (segment (start 133.35 44.45) (end 137.16 44.45) (width 1) (layer "F.Cu") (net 2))
 (segment (start 130.225489 45.094511) (end 131.4 43.92) (width 0.25) (layer "B.Cu") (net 2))
 (segment (start 127.7952 45.6868) (end 128.387489 45.094511) (width 0.25) (layer "B.Cu") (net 2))
 (segment (start 128.387489 45.094511) (end 130.225489 45.094511) (width 0.25) (layer "B.Cu") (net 2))
 (segment (start 125.7196 45.6868) (end 127.7952 45.6868) (width 0.25) (layer "B.Cu") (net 2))
 (segment (start 133.35 43.18) (end 132.914999 42.744999) (width 0.25) (layer "F.Cu") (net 1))
 (segment (start 133.35 43.18) (end 137.16 43.18) (width 1) (layer "F.Cu") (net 1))
 (segment (start 141.055012 44.5) (end 144.4 44.5) (width 0.25) (layer "F.Cu") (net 1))
 (segment (start 129.975001 42.744999) (end 129.54 43.18) (width 0.25) (layer "F.Cu") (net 1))
 (segment (start 137.16 43.18) (end 139.735012 43.18) (width 0.25) (layer "F.Cu") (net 1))
 (segment (start 144.4 44.5) (end 146.1 44.5) (width 0.25) (layer "F.Cu") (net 1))
 (segment (start 139.735012 43.18) (end 141.055012 44.5) (width 0.25) (layer "F.Cu") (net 1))
 (segment (start 132.914999 42.744999) (end 129.975001 42.744999) (width 0.25) (layer "F.Cu") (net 1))
 (segment (start 129.54 43.24) (end 128.86 43.92) (width 0.25) (layer "F.Cu") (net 1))
 (segment (start 129.54 43.18) (end 129.54 43.24) (width 0.25) (layer "F.Cu") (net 1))
 (segment (start 128.1932 44.5868) (end 128.86 43.92) (width 0.25) (layer "B.Cu") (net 1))
 (segment (start 125.7196 44.5868) (end 128.1932 44.5868) (width 0.25) (layer "B.Cu") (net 1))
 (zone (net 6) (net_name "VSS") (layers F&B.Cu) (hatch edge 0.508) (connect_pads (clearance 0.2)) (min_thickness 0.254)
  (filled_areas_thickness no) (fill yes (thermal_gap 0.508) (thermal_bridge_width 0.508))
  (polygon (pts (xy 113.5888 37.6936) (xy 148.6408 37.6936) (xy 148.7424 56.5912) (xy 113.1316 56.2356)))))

